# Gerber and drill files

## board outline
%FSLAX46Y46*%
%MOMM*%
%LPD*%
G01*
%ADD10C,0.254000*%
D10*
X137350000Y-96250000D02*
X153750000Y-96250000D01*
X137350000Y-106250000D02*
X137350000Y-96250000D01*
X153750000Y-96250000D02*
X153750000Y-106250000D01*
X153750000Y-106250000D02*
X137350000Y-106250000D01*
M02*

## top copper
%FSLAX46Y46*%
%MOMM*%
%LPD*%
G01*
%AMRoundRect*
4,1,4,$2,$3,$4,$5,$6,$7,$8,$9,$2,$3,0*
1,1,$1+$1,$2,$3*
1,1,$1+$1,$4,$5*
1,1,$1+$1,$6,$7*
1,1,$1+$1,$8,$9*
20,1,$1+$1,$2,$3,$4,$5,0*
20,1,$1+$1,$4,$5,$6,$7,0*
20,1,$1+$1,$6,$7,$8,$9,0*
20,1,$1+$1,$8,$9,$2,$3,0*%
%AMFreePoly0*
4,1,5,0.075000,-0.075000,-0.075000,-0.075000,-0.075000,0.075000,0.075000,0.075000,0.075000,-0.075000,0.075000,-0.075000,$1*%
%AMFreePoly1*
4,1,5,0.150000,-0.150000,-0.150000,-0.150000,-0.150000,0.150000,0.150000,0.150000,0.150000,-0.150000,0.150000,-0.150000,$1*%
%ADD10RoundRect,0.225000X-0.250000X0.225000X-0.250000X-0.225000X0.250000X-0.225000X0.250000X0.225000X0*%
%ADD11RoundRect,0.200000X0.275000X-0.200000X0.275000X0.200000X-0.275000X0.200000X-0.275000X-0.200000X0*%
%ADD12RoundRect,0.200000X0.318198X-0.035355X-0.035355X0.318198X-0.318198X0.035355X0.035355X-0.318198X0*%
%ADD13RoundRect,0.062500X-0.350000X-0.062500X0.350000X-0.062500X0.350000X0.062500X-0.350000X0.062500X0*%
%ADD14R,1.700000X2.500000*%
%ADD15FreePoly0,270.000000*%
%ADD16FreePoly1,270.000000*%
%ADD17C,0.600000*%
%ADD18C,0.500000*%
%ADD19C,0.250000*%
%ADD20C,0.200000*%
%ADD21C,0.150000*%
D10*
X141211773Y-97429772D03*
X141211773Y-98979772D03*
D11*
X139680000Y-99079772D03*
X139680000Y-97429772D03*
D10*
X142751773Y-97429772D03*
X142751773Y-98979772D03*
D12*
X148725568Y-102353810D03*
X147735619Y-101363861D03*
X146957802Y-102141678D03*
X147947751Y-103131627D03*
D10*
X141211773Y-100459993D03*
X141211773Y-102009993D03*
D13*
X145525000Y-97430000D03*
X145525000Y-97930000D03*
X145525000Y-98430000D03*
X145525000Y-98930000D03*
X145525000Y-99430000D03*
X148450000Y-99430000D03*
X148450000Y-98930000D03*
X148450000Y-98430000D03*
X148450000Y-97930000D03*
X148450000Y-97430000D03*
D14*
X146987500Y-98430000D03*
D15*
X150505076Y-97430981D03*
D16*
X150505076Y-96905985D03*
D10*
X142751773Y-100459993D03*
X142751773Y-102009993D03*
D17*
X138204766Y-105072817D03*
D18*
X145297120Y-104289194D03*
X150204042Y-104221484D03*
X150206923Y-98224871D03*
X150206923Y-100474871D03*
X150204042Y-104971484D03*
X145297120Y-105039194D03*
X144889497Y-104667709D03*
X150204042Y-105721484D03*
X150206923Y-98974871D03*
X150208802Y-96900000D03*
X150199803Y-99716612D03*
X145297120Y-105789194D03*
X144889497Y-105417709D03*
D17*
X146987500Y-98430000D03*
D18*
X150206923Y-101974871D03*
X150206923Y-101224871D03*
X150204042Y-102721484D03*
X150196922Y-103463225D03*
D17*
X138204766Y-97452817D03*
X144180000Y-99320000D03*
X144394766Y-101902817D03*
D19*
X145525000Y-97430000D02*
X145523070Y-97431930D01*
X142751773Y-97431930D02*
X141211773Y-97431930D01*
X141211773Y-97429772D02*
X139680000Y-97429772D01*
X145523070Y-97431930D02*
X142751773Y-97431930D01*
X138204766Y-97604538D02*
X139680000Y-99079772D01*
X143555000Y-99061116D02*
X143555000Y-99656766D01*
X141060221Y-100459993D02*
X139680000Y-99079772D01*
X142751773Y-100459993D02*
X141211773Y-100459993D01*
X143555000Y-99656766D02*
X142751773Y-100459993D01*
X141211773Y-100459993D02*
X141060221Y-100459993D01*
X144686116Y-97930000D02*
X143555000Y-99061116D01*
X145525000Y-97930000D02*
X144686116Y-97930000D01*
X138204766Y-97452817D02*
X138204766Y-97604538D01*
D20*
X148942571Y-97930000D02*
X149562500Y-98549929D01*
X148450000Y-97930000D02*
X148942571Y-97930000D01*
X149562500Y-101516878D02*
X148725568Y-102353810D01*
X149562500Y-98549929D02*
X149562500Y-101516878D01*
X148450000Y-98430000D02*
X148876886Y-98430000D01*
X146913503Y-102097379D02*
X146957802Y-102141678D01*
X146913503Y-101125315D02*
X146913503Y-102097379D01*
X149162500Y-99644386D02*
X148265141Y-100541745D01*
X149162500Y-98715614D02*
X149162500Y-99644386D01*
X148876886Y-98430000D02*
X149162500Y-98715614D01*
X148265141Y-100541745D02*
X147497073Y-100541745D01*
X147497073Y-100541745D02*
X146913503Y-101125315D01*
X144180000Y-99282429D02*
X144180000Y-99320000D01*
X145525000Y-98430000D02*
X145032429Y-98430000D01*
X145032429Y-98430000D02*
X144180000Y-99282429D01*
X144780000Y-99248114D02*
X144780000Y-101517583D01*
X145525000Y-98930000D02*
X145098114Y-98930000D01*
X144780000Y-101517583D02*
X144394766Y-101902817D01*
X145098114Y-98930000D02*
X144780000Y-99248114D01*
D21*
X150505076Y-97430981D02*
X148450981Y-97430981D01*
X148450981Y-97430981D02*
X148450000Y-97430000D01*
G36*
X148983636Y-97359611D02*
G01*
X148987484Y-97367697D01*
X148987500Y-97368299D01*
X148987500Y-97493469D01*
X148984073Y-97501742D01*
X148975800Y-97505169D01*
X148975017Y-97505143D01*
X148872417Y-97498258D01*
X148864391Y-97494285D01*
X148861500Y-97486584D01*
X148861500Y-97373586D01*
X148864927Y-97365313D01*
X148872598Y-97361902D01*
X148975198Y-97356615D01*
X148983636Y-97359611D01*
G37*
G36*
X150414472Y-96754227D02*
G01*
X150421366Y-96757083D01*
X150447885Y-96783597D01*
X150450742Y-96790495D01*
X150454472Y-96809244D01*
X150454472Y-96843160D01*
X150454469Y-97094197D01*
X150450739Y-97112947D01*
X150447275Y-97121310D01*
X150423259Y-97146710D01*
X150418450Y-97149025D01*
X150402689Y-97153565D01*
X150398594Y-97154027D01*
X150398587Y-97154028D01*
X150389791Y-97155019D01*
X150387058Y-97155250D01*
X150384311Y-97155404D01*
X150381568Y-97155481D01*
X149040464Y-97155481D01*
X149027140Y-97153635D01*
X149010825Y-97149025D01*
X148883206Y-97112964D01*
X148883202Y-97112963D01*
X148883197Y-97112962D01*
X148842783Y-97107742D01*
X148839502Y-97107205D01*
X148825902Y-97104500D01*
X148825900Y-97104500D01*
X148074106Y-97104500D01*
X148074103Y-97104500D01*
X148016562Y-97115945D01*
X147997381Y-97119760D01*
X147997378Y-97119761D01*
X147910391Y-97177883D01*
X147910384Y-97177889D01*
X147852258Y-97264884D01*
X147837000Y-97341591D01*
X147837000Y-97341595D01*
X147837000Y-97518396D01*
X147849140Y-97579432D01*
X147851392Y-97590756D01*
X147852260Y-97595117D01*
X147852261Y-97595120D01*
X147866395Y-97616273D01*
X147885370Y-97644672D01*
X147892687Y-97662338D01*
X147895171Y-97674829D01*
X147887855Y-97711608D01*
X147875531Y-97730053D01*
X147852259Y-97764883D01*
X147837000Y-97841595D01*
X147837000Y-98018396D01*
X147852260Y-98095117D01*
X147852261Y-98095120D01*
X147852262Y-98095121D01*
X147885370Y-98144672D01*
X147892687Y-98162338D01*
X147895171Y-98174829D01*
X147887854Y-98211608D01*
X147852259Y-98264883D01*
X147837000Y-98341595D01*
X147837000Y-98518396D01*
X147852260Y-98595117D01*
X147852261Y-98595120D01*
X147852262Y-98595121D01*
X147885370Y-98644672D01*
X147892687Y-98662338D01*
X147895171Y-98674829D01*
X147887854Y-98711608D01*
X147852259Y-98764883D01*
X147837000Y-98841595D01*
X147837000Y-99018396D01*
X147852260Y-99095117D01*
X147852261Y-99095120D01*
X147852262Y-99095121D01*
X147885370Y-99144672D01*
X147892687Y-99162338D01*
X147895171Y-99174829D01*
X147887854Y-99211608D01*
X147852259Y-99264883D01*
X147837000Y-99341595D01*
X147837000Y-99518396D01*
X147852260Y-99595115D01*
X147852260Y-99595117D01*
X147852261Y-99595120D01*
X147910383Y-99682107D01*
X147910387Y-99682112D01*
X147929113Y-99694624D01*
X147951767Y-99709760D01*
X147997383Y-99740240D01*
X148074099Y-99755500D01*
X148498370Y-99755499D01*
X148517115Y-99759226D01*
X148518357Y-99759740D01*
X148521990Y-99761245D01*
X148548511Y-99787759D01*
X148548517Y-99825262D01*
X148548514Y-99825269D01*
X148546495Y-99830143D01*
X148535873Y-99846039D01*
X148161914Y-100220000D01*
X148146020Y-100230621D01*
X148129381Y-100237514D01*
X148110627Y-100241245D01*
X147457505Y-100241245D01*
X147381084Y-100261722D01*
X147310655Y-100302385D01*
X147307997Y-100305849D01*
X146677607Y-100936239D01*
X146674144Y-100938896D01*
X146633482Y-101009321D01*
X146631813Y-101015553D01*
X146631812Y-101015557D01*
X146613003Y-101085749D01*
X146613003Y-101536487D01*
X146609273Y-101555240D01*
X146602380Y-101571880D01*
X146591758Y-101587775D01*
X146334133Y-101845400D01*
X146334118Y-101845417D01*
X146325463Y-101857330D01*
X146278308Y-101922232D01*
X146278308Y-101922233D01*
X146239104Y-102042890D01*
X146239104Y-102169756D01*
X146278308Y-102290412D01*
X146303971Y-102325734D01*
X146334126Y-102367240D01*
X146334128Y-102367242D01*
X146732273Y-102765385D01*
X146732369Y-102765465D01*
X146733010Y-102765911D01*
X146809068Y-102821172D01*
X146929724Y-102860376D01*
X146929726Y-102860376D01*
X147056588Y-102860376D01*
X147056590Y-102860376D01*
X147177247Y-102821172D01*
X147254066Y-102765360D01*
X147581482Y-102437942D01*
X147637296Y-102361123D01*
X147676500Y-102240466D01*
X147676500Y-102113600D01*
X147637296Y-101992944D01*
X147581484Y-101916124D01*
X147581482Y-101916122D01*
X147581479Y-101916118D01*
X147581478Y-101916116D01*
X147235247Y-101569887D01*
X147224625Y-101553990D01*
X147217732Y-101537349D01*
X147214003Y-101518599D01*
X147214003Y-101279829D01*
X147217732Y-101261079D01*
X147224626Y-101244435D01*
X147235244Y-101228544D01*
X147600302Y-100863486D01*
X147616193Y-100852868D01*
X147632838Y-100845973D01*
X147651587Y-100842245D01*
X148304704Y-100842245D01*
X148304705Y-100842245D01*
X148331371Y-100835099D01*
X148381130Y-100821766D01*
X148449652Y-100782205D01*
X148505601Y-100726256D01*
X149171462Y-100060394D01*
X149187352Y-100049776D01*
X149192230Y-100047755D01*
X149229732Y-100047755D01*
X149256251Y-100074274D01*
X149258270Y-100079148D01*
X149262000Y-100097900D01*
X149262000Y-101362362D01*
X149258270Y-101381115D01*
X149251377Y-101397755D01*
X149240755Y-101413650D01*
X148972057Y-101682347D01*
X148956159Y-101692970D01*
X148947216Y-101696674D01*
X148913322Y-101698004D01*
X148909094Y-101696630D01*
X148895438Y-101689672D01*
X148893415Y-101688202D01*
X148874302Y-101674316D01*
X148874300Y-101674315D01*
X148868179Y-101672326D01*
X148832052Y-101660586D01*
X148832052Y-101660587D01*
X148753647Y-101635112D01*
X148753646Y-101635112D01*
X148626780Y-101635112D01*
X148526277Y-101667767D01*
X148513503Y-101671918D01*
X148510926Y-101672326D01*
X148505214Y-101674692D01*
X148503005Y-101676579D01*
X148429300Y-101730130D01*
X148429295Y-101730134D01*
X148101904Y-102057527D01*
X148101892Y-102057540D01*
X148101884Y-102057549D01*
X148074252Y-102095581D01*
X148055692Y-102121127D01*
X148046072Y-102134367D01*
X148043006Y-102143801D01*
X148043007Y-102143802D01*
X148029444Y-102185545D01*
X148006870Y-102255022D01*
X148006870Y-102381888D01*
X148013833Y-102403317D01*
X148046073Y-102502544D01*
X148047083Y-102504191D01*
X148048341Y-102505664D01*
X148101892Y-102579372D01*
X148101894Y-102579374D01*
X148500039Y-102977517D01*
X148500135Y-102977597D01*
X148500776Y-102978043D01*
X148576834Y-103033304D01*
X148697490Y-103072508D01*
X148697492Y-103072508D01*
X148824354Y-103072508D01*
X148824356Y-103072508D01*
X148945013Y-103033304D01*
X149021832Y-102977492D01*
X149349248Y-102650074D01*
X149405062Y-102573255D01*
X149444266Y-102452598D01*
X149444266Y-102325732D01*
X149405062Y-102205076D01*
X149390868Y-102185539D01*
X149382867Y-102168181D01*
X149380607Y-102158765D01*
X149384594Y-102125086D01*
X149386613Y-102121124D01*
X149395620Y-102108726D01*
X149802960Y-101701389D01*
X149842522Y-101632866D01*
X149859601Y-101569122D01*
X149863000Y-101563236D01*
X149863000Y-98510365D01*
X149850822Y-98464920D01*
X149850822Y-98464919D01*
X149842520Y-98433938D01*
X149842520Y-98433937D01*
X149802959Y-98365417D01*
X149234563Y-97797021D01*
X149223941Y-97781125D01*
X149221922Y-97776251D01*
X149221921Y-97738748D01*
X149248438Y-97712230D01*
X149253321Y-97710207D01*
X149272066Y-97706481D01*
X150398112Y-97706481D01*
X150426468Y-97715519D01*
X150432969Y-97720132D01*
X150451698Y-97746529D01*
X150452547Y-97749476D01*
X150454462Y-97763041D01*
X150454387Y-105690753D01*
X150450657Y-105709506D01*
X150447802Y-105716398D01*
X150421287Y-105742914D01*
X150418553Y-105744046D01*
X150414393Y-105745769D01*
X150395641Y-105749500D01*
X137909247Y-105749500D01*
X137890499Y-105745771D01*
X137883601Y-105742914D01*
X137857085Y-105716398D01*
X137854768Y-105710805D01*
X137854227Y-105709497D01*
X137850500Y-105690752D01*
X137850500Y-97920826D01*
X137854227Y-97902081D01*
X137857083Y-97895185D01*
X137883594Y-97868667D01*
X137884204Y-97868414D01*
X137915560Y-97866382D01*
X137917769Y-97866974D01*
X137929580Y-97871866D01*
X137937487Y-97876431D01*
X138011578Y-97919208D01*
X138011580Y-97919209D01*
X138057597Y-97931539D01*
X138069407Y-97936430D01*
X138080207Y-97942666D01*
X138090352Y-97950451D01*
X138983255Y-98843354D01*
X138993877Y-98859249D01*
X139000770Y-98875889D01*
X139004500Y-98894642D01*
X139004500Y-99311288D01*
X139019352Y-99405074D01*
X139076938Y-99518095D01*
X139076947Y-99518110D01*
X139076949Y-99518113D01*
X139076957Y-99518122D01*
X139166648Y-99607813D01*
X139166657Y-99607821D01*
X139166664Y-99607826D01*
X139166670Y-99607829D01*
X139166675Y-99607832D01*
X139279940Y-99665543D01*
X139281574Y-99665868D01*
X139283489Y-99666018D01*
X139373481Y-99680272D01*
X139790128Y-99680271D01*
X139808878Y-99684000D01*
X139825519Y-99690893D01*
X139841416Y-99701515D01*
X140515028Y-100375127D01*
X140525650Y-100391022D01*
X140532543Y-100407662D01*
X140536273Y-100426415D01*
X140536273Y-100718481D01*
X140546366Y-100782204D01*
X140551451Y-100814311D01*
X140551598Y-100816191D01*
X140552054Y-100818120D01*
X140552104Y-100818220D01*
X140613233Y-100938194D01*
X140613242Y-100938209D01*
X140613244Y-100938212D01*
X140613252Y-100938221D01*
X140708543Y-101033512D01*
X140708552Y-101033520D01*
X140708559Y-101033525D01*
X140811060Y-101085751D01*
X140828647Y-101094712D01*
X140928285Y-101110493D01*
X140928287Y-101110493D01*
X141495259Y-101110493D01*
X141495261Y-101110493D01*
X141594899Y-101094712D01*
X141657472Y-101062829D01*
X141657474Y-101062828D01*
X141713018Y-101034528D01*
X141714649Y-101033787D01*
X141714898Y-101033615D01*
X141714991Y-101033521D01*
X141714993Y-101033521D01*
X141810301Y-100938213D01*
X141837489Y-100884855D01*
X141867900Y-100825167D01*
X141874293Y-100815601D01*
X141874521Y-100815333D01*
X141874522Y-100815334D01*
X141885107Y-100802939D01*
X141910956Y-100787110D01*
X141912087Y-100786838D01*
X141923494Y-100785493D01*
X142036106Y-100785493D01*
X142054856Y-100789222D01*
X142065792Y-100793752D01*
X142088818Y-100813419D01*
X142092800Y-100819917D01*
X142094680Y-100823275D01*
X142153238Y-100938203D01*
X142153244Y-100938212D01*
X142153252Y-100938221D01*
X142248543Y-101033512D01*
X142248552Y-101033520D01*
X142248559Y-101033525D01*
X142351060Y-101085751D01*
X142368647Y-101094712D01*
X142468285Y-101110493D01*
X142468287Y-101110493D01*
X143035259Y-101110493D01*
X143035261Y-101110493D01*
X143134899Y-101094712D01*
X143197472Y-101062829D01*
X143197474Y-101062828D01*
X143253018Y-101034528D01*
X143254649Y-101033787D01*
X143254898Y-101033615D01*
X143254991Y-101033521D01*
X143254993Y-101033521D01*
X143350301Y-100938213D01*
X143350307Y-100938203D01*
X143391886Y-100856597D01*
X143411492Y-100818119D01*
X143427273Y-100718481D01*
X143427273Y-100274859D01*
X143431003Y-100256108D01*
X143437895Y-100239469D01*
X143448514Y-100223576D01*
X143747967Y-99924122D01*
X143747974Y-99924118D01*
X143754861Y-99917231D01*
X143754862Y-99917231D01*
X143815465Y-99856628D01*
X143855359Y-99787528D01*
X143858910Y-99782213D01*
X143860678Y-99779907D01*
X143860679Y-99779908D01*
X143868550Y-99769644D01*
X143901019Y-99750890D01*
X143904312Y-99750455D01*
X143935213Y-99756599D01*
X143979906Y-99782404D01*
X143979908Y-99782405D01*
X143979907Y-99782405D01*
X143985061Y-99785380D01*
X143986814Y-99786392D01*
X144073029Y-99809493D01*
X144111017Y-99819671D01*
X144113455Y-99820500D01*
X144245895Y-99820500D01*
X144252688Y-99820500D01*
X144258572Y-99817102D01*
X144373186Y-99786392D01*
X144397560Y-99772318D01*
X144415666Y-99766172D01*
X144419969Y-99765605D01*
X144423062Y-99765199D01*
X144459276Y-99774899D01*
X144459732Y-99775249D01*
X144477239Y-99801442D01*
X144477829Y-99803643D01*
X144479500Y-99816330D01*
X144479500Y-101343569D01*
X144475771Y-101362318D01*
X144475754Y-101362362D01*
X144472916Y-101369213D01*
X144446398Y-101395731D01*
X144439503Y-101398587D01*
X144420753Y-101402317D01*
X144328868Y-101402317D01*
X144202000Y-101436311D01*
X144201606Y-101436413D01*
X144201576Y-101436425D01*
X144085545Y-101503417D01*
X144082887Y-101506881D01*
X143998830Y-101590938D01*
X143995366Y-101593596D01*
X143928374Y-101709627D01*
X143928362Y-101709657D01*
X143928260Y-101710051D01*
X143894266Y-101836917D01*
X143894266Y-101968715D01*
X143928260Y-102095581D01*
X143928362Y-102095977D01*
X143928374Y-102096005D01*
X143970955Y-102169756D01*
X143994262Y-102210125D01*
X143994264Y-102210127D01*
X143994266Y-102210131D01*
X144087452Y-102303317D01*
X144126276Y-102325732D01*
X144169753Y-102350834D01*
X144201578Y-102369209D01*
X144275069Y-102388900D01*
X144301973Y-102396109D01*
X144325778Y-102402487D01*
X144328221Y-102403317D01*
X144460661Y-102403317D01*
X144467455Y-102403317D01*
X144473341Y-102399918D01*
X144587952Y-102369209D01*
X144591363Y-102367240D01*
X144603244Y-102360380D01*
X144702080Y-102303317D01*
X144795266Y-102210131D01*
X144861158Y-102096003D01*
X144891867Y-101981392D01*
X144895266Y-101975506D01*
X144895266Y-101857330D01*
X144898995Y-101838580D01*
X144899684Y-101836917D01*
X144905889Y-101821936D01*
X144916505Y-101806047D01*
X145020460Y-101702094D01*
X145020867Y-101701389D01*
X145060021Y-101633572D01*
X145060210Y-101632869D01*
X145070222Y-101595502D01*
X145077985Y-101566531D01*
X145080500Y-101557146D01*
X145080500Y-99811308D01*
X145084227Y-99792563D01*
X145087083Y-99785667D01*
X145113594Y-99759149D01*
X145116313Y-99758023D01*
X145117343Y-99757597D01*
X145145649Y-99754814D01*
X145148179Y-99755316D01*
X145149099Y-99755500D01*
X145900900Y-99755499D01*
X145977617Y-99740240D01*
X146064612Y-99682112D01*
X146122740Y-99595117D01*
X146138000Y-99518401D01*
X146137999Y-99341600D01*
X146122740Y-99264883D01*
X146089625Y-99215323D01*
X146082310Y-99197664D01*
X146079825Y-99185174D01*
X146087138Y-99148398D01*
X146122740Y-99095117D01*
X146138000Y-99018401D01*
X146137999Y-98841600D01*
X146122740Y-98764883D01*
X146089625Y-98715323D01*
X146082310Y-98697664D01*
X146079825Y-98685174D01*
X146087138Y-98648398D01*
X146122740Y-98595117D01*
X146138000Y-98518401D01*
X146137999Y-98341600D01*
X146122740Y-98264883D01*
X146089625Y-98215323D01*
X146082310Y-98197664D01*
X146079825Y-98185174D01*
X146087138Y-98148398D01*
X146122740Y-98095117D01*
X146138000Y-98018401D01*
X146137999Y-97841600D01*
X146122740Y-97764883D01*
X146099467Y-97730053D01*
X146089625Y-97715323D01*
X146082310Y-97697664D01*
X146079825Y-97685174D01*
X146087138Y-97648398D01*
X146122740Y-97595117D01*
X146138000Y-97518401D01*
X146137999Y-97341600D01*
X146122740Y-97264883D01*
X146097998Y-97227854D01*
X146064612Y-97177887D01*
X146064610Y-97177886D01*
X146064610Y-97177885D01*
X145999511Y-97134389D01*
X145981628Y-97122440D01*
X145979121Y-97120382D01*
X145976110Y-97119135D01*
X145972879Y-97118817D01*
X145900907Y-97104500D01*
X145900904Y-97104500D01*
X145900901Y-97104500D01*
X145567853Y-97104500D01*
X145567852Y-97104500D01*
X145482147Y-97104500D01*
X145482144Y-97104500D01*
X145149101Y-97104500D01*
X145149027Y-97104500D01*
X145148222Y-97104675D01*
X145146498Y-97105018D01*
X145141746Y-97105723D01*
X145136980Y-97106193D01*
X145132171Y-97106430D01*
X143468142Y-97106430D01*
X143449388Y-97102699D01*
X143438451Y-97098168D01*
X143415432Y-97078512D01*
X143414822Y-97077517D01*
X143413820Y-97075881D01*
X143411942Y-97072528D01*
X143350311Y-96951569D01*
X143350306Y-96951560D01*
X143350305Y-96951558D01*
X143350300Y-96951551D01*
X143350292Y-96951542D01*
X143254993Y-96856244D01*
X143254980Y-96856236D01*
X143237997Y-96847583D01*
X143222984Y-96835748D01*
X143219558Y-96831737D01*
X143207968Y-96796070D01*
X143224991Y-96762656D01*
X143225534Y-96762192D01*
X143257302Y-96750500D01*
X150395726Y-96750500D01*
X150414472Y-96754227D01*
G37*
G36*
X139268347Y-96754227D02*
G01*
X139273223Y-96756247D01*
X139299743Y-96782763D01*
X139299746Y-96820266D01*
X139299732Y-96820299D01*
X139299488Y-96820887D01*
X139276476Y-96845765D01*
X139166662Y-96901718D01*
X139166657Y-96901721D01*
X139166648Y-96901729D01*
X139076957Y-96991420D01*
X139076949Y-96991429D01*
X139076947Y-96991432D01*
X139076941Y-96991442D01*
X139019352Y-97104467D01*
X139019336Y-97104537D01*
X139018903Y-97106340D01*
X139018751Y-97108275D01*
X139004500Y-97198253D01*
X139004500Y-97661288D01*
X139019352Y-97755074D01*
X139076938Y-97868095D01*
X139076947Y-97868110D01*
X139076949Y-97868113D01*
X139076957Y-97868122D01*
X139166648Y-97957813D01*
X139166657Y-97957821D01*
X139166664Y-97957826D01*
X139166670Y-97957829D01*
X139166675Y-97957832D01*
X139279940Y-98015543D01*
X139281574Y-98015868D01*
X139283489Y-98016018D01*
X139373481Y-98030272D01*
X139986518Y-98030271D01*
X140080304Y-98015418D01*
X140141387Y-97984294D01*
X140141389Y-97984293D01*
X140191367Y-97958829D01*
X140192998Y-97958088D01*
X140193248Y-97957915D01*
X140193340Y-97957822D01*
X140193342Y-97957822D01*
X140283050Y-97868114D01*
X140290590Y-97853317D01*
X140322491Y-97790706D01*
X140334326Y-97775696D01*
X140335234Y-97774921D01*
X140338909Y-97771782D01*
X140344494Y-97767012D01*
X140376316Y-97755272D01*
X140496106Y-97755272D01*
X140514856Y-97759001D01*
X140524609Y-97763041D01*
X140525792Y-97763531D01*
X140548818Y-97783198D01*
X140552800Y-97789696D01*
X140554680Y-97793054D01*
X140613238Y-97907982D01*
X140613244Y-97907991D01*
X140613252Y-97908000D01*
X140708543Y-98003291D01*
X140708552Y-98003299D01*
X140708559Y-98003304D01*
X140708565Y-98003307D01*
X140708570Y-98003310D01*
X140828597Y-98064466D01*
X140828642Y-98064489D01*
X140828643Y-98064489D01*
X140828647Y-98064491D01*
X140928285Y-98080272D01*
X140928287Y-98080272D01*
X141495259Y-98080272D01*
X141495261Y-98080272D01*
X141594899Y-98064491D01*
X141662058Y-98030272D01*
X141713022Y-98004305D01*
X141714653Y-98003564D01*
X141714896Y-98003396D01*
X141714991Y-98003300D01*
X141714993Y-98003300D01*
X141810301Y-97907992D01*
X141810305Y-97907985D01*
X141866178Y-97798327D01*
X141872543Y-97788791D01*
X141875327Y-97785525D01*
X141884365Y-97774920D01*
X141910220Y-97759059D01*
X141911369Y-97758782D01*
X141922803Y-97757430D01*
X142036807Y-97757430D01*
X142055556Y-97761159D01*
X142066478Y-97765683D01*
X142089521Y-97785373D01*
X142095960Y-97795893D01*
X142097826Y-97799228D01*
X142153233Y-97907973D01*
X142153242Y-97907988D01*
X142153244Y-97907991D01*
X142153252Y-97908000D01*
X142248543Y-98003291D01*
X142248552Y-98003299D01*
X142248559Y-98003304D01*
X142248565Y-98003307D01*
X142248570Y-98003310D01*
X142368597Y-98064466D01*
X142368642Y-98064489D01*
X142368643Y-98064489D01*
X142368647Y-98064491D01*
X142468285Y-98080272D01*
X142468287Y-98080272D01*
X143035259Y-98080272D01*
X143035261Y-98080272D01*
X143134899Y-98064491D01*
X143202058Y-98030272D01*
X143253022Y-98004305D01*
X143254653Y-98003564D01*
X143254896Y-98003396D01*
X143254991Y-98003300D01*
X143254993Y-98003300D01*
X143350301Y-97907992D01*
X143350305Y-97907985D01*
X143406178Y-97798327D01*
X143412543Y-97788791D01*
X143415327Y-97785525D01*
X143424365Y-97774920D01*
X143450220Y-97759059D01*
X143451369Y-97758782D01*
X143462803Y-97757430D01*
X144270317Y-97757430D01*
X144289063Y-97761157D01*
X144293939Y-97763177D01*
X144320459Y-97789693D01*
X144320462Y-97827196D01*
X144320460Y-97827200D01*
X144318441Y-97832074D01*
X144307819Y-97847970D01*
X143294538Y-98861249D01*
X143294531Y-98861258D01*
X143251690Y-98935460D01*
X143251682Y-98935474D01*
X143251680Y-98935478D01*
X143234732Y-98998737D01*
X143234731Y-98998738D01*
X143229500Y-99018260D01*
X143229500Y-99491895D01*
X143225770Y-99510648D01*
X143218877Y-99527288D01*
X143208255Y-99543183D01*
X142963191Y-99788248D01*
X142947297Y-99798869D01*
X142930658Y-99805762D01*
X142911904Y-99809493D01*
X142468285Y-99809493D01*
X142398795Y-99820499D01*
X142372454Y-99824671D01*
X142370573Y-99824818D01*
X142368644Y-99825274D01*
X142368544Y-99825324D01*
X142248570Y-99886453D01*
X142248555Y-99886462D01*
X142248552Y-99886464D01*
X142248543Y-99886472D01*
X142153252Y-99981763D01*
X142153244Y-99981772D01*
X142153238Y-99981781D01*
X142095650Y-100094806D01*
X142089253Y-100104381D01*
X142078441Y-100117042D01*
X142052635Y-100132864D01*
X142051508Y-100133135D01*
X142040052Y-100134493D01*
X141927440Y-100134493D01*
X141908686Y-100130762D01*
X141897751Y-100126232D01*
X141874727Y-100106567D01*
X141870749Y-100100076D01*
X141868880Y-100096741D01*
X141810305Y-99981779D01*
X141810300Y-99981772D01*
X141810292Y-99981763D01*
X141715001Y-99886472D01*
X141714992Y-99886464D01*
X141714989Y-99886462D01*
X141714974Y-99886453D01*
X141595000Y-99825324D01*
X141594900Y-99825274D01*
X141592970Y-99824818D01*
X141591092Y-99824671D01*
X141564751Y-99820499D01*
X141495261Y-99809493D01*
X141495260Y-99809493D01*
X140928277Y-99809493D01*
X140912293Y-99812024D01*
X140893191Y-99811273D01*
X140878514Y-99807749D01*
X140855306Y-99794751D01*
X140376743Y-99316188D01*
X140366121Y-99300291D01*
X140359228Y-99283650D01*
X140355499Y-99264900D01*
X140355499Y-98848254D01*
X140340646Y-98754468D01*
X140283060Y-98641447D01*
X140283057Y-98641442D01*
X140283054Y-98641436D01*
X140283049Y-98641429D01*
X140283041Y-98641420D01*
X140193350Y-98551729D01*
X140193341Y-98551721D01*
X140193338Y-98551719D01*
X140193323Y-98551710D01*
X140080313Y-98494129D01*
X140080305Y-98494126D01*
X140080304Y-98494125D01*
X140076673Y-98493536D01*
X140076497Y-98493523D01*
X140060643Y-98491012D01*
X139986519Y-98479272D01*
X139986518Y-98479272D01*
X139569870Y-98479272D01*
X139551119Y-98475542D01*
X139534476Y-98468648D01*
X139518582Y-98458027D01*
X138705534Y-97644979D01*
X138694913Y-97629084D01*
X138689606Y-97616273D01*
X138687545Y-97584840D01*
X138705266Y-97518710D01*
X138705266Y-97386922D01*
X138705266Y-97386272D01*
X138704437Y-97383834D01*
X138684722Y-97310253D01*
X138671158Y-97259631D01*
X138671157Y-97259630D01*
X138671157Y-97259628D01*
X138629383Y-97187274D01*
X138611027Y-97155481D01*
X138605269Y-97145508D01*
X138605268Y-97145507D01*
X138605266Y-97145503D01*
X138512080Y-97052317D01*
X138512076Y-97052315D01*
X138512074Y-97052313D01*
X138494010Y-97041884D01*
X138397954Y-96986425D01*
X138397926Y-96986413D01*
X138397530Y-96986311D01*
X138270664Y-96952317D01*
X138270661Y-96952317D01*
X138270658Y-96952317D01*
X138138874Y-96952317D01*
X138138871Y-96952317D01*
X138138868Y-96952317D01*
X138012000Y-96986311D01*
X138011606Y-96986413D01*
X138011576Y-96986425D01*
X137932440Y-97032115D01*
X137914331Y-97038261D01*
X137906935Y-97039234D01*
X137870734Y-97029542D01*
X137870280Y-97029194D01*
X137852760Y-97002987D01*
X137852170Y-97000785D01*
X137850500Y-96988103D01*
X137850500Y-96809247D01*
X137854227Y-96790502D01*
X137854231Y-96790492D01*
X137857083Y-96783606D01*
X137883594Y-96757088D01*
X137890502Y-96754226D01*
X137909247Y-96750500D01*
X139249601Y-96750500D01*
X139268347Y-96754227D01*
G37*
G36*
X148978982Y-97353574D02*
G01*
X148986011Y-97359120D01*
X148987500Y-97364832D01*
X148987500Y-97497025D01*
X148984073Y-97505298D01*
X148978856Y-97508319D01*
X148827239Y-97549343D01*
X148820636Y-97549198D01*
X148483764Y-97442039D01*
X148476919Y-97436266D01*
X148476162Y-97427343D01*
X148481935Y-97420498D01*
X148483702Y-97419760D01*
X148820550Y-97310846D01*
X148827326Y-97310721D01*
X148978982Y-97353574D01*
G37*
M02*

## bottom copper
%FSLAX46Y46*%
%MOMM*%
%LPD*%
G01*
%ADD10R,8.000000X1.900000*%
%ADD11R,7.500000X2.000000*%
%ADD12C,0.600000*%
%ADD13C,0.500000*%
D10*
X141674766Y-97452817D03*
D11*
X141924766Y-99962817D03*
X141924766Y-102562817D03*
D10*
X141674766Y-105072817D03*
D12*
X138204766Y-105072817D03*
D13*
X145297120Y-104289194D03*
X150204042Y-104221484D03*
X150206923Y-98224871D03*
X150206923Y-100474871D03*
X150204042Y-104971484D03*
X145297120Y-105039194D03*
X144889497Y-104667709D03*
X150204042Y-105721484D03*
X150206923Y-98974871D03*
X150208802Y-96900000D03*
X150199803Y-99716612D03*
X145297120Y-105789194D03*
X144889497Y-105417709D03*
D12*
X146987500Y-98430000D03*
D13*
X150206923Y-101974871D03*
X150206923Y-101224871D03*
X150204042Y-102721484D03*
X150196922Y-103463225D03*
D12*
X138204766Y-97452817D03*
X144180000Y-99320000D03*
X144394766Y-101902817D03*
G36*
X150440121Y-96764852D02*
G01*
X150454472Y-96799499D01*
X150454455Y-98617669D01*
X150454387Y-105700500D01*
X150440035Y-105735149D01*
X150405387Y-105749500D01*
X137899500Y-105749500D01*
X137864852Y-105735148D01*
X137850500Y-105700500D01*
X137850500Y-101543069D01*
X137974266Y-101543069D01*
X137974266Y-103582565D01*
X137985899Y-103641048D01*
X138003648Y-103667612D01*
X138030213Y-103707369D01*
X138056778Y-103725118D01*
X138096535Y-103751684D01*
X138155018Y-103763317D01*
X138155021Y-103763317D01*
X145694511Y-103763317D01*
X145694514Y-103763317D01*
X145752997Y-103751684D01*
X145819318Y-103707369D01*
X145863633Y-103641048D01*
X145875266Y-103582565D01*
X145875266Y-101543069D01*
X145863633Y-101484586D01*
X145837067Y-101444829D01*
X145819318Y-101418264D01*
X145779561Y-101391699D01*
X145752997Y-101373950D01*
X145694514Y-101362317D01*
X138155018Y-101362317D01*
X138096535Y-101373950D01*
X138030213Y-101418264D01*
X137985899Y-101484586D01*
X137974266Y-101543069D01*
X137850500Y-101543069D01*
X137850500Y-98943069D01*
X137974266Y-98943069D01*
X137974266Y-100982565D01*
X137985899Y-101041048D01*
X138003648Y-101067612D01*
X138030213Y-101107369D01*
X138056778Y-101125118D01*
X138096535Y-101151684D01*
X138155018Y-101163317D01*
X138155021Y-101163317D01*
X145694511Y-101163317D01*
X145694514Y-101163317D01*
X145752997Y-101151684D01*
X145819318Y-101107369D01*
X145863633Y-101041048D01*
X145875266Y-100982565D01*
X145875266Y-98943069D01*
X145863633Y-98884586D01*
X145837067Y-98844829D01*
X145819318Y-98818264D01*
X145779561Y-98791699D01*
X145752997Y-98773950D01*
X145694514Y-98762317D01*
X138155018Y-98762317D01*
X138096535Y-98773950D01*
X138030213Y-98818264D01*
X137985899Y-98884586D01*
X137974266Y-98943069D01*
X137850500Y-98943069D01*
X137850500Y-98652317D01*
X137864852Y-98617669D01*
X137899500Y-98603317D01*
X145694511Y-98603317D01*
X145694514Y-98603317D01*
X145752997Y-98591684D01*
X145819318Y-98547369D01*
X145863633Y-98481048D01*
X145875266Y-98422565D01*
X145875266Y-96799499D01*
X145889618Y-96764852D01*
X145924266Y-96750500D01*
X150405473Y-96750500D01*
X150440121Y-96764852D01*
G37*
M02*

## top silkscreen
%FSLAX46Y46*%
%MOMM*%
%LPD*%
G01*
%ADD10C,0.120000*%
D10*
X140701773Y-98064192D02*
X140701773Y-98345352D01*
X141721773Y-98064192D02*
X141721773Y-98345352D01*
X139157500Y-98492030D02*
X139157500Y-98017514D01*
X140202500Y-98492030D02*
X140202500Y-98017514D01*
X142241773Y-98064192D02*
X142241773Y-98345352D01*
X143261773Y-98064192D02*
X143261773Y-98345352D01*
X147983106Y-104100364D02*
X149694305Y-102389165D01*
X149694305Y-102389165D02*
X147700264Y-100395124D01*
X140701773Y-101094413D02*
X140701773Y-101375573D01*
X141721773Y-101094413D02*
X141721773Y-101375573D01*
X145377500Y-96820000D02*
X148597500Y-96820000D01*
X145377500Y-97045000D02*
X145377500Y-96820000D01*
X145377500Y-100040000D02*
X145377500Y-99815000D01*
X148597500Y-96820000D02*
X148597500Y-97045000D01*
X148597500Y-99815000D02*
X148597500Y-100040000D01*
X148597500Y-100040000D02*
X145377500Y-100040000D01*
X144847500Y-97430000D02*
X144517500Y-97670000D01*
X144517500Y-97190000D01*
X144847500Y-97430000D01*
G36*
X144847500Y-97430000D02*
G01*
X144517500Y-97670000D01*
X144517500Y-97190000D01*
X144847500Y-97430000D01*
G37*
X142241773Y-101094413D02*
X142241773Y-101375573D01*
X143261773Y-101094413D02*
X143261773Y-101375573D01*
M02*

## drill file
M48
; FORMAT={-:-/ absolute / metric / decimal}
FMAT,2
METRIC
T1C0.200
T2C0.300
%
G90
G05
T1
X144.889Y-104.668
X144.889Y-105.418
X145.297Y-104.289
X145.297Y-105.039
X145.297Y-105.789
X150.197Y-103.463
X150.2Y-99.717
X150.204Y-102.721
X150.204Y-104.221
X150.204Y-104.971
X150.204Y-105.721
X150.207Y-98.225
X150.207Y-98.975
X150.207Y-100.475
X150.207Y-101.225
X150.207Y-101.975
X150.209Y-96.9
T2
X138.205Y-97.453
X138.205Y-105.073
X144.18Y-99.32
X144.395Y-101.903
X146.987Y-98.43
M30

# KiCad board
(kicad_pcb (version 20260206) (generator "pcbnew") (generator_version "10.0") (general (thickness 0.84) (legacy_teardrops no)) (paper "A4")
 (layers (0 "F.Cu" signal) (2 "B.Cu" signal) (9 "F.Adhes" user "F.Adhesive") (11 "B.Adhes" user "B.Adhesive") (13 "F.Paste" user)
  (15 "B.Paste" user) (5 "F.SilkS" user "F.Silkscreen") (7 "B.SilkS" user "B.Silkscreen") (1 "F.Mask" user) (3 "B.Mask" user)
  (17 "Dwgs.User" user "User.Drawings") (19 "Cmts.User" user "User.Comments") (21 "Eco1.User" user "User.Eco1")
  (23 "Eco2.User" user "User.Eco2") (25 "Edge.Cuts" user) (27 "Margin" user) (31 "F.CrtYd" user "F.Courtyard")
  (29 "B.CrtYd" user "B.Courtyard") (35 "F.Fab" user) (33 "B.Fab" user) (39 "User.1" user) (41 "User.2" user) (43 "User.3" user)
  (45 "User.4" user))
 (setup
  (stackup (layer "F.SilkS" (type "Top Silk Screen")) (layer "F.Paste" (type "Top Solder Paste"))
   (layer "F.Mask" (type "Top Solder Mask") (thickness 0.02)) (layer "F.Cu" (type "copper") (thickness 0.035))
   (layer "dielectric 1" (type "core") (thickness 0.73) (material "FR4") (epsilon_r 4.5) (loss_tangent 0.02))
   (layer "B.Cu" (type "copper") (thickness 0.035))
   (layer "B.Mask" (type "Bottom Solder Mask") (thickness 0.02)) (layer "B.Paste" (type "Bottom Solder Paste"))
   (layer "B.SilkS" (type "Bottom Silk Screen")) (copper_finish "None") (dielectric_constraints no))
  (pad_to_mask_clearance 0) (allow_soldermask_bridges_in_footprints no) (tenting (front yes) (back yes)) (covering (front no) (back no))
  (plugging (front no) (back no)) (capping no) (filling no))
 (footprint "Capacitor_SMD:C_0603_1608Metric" (layer "F.Cu") (at 141.211773 98.204772 -90)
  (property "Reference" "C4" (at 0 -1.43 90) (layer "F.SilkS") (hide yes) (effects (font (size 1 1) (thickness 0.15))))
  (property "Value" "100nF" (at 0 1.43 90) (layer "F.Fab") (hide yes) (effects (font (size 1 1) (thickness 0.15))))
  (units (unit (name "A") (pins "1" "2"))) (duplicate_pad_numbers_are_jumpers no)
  (fp_line (start -0.14058 0.51) (end 0.14058 0.51) (stroke (width 0.12) (type solid)) (layer "F.SilkS"))
  (fp_line (start -0.14058 -0.51) (end 0.14058 -0.51) (stroke (width 0.12) (type solid)) (layer "F.SilkS"))
  (pad "1" smd roundrect (at -0.775 0 270) (size 0.9 0.95) (layers "F.Cu" "F.Mask" "F.Paste") (roundrect_rratio 0.25) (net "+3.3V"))
  (pad "2" smd roundrect (at 0.775 0 270) (size 0.9 0.95) (layers "F.Cu" "F.Mask" "F.Paste") (roundrect_rratio 0.25) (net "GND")))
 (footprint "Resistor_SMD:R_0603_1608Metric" (layer "F.Cu") (at 139.68 98.254772 90)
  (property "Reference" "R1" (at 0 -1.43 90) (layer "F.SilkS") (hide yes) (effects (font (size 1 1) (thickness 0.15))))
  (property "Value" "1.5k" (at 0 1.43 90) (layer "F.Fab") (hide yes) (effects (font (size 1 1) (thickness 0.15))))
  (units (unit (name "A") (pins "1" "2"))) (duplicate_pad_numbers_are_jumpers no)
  (fp_line (start -0.237258 -0.5225) (end 0.237258 -0.5225) (stroke (width 0.12) (type solid)) (layer "F.SilkS"))
  (fp_line (start -0.237258 0.5225) (end 0.237258 0.5225) (stroke (width 0.12) (type solid)) (layer "F.SilkS"))
  (pad "1" smd roundrect (at -0.825 0 90) (size 0.8 0.95) (layers "F.Cu" "F.Mask" "F.Paste") (roundrect_rratio 0.25) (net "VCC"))
  (pad "2" smd roundrect (at 0.825 0 90) (size 0.8 0.95) (layers "F.Cu" "F.Mask" "F.Paste") (roundrect_rratio 0.25) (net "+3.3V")))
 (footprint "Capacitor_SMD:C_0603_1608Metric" (layer "F.Cu") (at 142.751773 98.204772 -90)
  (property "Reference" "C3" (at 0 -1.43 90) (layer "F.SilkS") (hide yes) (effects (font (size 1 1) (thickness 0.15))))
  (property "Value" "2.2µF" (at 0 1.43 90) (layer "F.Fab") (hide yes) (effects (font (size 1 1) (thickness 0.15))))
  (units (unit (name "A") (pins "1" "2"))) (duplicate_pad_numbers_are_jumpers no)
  (fp_line (start -0.14058 0.51) (end 0.14058 0.51) (stroke (width 0.12) (type solid)) (layer "F.SilkS"))
  (fp_line (start -0.14058 -0.51) (end 0.14058 -0.51) (stroke (width 0.12) (type solid)) (layer "F.SilkS"))
  (pad "1" smd roundrect (at -0.775 0 270) (size 0.9 0.95) (layers "F.Cu" "F.Mask" "F.Paste") (roundrect_rratio 0.25) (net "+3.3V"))
  (pad "2" smd roundrect (at 0.775 0 270) (size 0.9 0.95) (layers "F.Cu" "F.Mask" "F.Paste") (roundrect_rratio 0.25) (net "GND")))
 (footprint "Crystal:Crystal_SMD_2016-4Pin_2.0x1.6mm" (layer "F.Cu") (at 147.841685 102.247744 135)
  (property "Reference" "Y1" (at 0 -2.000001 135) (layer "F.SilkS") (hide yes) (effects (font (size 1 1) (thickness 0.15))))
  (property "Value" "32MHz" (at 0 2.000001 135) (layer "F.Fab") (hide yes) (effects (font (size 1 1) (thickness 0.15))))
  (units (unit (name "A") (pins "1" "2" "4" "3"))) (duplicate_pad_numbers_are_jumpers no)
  (fp_line (start -1.41 -1.21) (end -1.41 1.21) (stroke (width 0.12) (type solid)) (layer "F.SilkS"))
  (fp_line (start -1.41 1.21) (end 1.41 1.21) (stroke (width 0.12) (type solid)) (layer "F.SilkS"))
  (pad "1" smd roundrect (at -0.7 0.55 135) (size 0.9 0.8) (layers "F.Cu" "F.Mask" "F.Paste") (roundrect_rratio 0.25) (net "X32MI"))
  (pad "2" smd roundrect (at 0.7 0.55 135) (size 0.9 0.8) (layers "F.Cu" "F.Mask" "F.Paste") (roundrect_rratio 0.25) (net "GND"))
  (pad "3" smd roundrect (at 0.7 -0.55 135) (size 0.9 0.8) (layers "F.Cu" "F.Mask" "F.Paste") (roundrect_rratio 0.25) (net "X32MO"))
  (pad "4" smd roundrect (at -0.7 -0.55 135) (size 0.9 0.8) (layers "F.Cu" "F.Mask" "F.Paste") (roundrect_rratio 0.25) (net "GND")))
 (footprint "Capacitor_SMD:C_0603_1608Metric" (layer "F.Cu") (at 141.211773 101.234993 -90)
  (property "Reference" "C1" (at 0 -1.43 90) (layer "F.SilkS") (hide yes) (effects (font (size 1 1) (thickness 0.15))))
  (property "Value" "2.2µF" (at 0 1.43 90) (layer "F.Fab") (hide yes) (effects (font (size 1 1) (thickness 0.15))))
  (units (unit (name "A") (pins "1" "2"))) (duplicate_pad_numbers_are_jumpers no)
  (fp_line (start -0.14058 0.51) (end 0.14058 0.51) (stroke (width 0.12) (type solid)) (layer "F.SilkS"))
  (fp_line (start -0.14058 -0.51) (end 0.14058 -0.51) (stroke (width 0.12) (type solid)) (layer "F.SilkS"))
  (pad "1" smd roundrect (at -0.775 0 270) (size 0.9 0.95) (layers "F.Cu" "F.Mask" "F.Paste") (roundrect_rratio 0.25) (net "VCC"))
  (pad "2" smd roundrect (at 0.775 0 270) (size 0.9 0.95) (layers "F.Cu" "F.Mask" "F.Paste") (roundrect_rratio 0.25) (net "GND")))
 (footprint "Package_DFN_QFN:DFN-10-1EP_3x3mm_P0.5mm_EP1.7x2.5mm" (layer "F.Cu") (at 146.9875 98.43)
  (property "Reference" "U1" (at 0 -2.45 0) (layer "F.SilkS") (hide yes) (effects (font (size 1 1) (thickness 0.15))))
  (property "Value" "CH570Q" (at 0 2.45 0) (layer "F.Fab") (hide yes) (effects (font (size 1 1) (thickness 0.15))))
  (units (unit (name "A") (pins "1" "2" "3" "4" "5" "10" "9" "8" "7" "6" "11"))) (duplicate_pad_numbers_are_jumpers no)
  (fp_line (start -1.61 -1.61) (end 1.61 -1.61) (stroke (width 0.12) (type solid)) (layer "F.SilkS"))
  (fp_line (start -1.61 -1.385) (end -1.61 -1.61) (stroke (width 0.12) (type solid)) (layer "F.SilkS"))
  (fp_line (start -1.61 1.61) (end -1.61 1.385) (stroke (width 0.12) (type solid)) (layer "F.SilkS"))
  (fp_line (start 1.61 -1.61) (end 1.61 -1.385) (stroke (width 0.12) (type solid)) (layer "F.SilkS"))
  (fp_line (start 1.61 1.385) (end 1.61 1.61) (stroke (width 0.12) (type solid)) (layer "F.SilkS"))
  (fp_line (start 1.61 1.61) (end -1.61 1.61) (stroke (width 0.12) (type solid)) (layer "F.SilkS"))
  (fp_poly (pts (xy -2.14 -1) (xy -2.47 -0.76) (xy -2.47 -1.24)) (stroke (width 0.12) (type solid)) (fill yes) (layer "F.SilkS"))
  (pad "" smd roundrect (at -0.425 -0.625) (size 0.69 1.01) (layers "F.Paste") (roundrect_rratio 0.25))
  (pad "" smd roundrect (at -0.425 0.625) (size 0.69 1.01) (layers "F.Paste") (roundrect_rratio 0.25))
  (pad "" smd roundrect (at 0.425 -0.625) (size 0.69 1.01) (layers "F.Paste") (roundrect_rratio 0.25))
  (pad "" smd roundrect (at 0.425 0.625) (size 0.69 1.01) (layers "F.Paste") (roundrect_rratio 0.25))
  (pad "1" smd roundrect (at -1.4625 -1) (size 0.825 0.25) (layers "F.Cu" "F.Mask" "F.Paste") (roundrect_rratio 0.25) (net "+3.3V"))
  (pad "2" smd roundrect (at -1.4625 -0.5) (size 0.825 0.25) (layers "F.Cu" "F.Mask" "F.Paste") (roundrect_rratio 0.25) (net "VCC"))
  (pad "3" smd roundrect (at -1.4625 0) (size 0.825 0.25) (layers "F.Cu" "F.Mask" "F.Paste") (roundrect_rratio 0.25) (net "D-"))
  (pad "4" smd roundrect (at -1.4625 0.5) (size 0.825 0.25) (layers "F.Cu" "F.Mask" "F.Paste") (roundrect_rratio 0.25) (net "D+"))
  (pad "5" smd roundrect (at -1.4625 1) (size 0.825 0.25) (layers "F.Cu" "F.Mask" "F.Paste") (roundrect_rratio 0.25)
   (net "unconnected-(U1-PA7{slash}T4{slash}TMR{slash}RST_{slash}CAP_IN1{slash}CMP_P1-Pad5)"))
  (pad "6" smd roundrect (at 1.4625 1) (size 0.825 0.25) (layers "F.Cu" "F.Mask" "F.Paste") (roundrect_rratio 0.25)
   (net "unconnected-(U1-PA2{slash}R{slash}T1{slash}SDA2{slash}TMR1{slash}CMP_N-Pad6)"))
  (pad "7" smd roundrect (at 1.4625 0.5) (size 0.825 0.25) (layers "F.Cu" "F.Mask" "F.Paste") (roundrect_rratio 0.25)
   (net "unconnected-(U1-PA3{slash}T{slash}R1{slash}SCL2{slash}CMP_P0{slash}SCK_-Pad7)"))
  (pad "8" smd roundrect (at 1.4625 0) (size 0.825 0.25) (layers "F.Cu" "F.Mask" "F.Paste") (roundrect_rratio 0.25) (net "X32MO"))
  (pad "9" smd roundrect (at 1.4625 -0.5) (size 0.825 0.25) (layers "F.Cu" "F.Mask" "F.Paste") (roundrect_rratio 0.25) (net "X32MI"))
  (pad "10" smd roundrect (at 1.4625 -1) (size 0.825 0.25) (layers "F.Cu" "F.Mask" "F.Paste") (roundrect_rratio 0.25) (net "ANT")
   (teardrops (best_length_ratio 0.5) (max_length 1) (best_width_ratio 1) (max_width 2) (curved_edges no) (filter_ratio 0.9) (enabled yes)
    (allow_two_segments yes) (prefer_zone_connections yes)))
  (pad "11" smd rect (at 0 0) (size 1.7 2.5) (layers "F.Cu" "F.Mask") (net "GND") (zone_connect 2)))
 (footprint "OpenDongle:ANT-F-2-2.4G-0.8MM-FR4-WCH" (layer "F.Cu") (at 151.800076 101.240981 -90)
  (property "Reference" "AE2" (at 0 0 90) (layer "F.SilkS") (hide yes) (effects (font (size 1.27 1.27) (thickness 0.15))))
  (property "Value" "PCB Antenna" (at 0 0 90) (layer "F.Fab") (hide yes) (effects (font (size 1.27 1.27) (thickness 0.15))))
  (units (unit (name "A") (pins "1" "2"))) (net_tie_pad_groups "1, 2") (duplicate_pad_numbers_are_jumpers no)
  (pad "1" smd custom (at -3.81 1.295 270) (size 0.15 0.15) (layers "F.Cu") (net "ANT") (solder_mask_margin 0.1016)
   (options (clearance outline) (anchor rect)) (primitives)
   (teardrops (best_length_ratio 0.5) (max_length 1) (best_width_ratio 1) (max_width 2) (curved_edges no) (filter_ratio 0.9) (enabled yes)
    (allow_two_segments yes) (prefer_zone_connections yes)))
  (pad "2" smd custom (at -4.334996 1.295 270) (size 0.3 0.3) (layers "F.Cu") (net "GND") (solder_mask_margin 0.1016)
   (options (clearance outline) (anchor rect)) (primitives)))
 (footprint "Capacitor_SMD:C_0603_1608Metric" (layer "F.Cu") (at 142.751773 101.234993 -90)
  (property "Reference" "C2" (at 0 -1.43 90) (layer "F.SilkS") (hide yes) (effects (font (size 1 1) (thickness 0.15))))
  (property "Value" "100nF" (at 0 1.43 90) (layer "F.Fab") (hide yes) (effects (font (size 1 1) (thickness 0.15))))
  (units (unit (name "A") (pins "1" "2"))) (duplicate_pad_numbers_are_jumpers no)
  (fp_line (start -0.14058 0.51) (end 0.14058 0.51) (stroke (width 0.12) (type solid)) (layer "F.SilkS"))
  (fp_line (start -0.14058 -0.51) (end 0.14058 -0.51) (stroke (width 0.12) (type solid)) (layer "F.SilkS"))
  (pad "1" smd roundrect (at -0.775 0 270) (size 0.9 0.95) (layers "F.Cu" "F.Mask" "F.Paste") (roundrect_rratio 0.25) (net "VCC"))
  (pad "2" smd roundrect (at 0.775 0 270) (size 0.9 0.95) (layers "F.Cu" "F.Mask" "F.Paste") (roundrect_rratio 0.25) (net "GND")))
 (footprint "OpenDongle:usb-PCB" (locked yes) (layer "B.Cu") (at 136.774766 101.262817 90)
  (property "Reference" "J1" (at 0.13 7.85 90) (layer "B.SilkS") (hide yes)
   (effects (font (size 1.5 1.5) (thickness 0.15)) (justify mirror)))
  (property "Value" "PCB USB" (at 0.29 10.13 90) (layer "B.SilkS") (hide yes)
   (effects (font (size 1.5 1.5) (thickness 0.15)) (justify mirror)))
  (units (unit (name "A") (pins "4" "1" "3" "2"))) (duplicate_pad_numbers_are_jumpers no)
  (pad "1" connect rect (at 3.81 4.9 90) (size 1.9 8) (layers "B.Cu" "B.Mask") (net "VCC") (thermal_bridge_angle 45))
  (pad "2" connect rect (at 1.3 5.15 90) (size 2 7.5) (layers "B.Cu" "B.Mask") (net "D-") (thermal_bridge_angle 45))
  (pad "3" connect rect (at -1.3 5.15 90) (size 2 7.5) (layers "B.Cu" "B.Mask") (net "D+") (thermal_bridge_angle 45))
  (pad "4" connect rect (at -3.81 4.9 90) (size 1.9 8) (layers "B.Cu" "B.Mask") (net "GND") (thermal_bridge_angle 45)))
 (gr_line (start 137.35 96.25) (end 153.75 96.25) (stroke (width 0.254) (type default)) (layer "Edge.Cuts"))
 (gr_line (start 137.35 106.25) (end 137.35 96.25) (stroke (width 0.254) (type default)) (layer "Edge.Cuts"))
 (gr_line (start 153.75 96.25) (end 153.75 106.25) (stroke (width 0.254) (type default)) (layer "Edge.Cuts"))
 (gr_line (start 153.75 106.25) (end 137.35 106.25) (stroke (width 0.254) (type default)) (locked yes) (layer "Edge.Cuts"))
 (segment (start 145.525 97.43) (end 145.52307 97.43193) (width 0.25) (layer "F.Cu") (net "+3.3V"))
 (segment (start 142.751773 97.43193) (end 141.211773 97.43193) (width 0.25) (layer "F.Cu") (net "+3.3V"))
 (segment (start 141.211773 97.429772) (end 139.68 97.429772) (width 0.25) (layer "F.Cu") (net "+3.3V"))
 (segment (start 145.52307 97.43193) (end 142.751773 97.43193) (width 0.25) (layer "F.Cu") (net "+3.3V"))
 (via (at 138.204766 105.072817) (size 0.6) (drill 0.3) (layers "F.Cu" "B.Cu") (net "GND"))
 (via (at 145.29712 104.289194) (size 0.5) (drill 0.2) (layers "F.Cu" "B.Cu") (free yes) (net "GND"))
 (via (at 150.204042 104.221484) (size 0.5) (drill 0.2) (layers "F.Cu" "B.Cu") (free yes) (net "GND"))
 (via (at 150.206923 98.224871) (size 0.5) (drill 0.2) (layers "F.Cu" "B.Cu") (free yes) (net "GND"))
 (via (at 150.206923 100.474871) (size 0.5) (drill 0.2) (layers "F.Cu" "B.Cu") (free yes) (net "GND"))
 (via (at 150.204042 104.971484) (size 0.5) (drill 0.2) (layers "F.Cu" "B.Cu") (free yes) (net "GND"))
 (via (at 145.29712 105.039194) (size 0.5) (drill 0.2) (layers "F.Cu" "B.Cu") (free yes) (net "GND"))
 (via (at 144.889497 104.667709) (size 0.5) (drill 0.2) (layers "F.Cu" "B.Cu") (free yes) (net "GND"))
 (via (at 150.204042 105.721484) (size 0.5) (drill 0.2) (layers "F.Cu" "B.Cu") (free yes) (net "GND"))
 (via (at 150.206923 98.974871) (size 0.5) (drill 0.2) (layers "F.Cu" "B.Cu") (free yes) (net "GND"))
 (via (at 150.208802 96.9) (size 0.5) (drill 0.2) (layers "F.Cu" "B.Cu") (free yes) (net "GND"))
 (via (at 150.199803 99.716612) (size 0.5) (drill 0.2) (layers "F.Cu" "B.Cu") (free yes) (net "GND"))
 (via (at 145.29712 105.789194) (size 0.5) (drill 0.2) (layers "F.Cu" "B.Cu") (free yes) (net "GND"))
 (via (at 144.889497 105.417709) (size 0.5) (drill 0.2) (layers "F.Cu" "B.Cu") (free yes) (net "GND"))
 (via (at 146.9875 98.43) (size 0.6) (drill 0.3) (layers "F.Cu" "B.Cu") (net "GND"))
 (via (at 150.206923 101.974871) (size 0.5) (drill 0.2) (layers "F.Cu" "B.Cu") (free yes) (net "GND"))
 (via (at 150.206923 101.224871) (size 0.5) (drill 0.2) (layers "F.Cu" "B.Cu") (free yes) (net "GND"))
 (via (at 150.204042 102.721484) (size 0.5) (drill 0.2) (layers "F.Cu" "B.Cu") (free yes) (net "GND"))
 (via (at 150.196922 103.463225) (size 0.5) (drill 0.2) (layers "F.Cu" "B.Cu") (free yes) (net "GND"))
 (segment (start 138.204766 97.604538) (end 139.68 99.079772) (width 0.25) (layer "F.Cu") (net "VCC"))
 (segment (start 143.555 99.061116) (end 143.555 99.656766) (width 0.25) (layer "F.Cu") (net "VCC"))
 (segment (start 141.060221 100.459993) (end 139.68 99.079772) (width 0.25) (layer "F.Cu") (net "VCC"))
 (segment (start 142.751773 100.459993) (end 141.211773 100.459993) (width 0.25) (layer "F.Cu") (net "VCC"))
 (segment (start 143.555 99.656766) (end 142.751773 100.459993) (width 0.25) (layer "F.Cu") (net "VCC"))
 (segment (start 141.211773 100.459993) (end 141.060221 100.459993) (width 0.25) (layer "F.Cu") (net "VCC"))
 (segment (start 144.686116 97.93) (end 143.555 99.061116) (width 0.25) (layer "F.Cu") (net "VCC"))
 (segment (start 145.525 97.93) (end 144.686116 97.93) (width 0.25) (layer "F.Cu") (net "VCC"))
 (segment (start 138.204766 97.452817) (end 138.204766 97.604538) (width 0.25) (layer "F.Cu") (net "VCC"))
 (via (at 138.204766 97.452817) (size 0.6) (drill 0.3) (layers "F.Cu" "B.Cu") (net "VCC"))
 (segment (start 148.942571 97.93) (end 149.5625 98.549929) (width 0.2) (layer "F.Cu") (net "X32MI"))
 (segment (start 148.45 97.93) (end 148.942571 97.93) (width 0.2) (layer "F.Cu") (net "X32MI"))
 (segment (start 149.5625 101.516878) (end 148.725568 102.35381) (width 0.2) (layer "F.Cu") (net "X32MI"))
 (segment (start 149.5625 98.549929) (end 149.5625 101.516878) (width 0.2) (layer "F.Cu") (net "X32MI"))
 (segment (start 148.45 98.43) (end 148.876886 98.43) (width 0.2) (layer "F.Cu") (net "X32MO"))
 (segment (start 146.913503 102.097379) (end 146.957802 102.141678) (width 0.2) (layer "F.Cu") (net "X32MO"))
 (segment (start 146.913503 101.125315) (end 146.913503 102.097379) (width 0.2) (layer "F.Cu") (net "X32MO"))
 (segment (start 149.1625 99.644386) (end 148.265141 100.541745) (width 0.2) (layer "F.Cu") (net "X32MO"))
 (segment (start 149.1625 98.715614) (end 149.1625 99.644386) (width 0.2) (layer "F.Cu") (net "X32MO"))
 (segment (start 148.876886 98.43) (end 149.1625 98.715614) (width 0.2) (layer "F.Cu") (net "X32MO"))
 (segment (start 148.265141 100.541745) (end 147.497073 100.541745) (width 0.2) (layer "F.Cu") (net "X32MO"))
 (segment (start 147.497073 100.541745) (end 146.913503 101.125315) (width 0.2) (layer "F.Cu") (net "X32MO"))
 (segment (start 144.18 99.282429) (end 144.18 99.32) (width 0.2) (layer "F.Cu") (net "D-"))
 (segment (start 145.525 98.43) (end 145.032429 98.43) (width 0.2) (layer "F.Cu") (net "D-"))
 (segment (start 145.032429 98.43) (end 144.18 99.282429) (width 0.2) (layer "F.Cu") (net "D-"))
 (via (at 144.18 99.32) (size 0.6) (drill 0.3) (layers "F.Cu" "B.Cu") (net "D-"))
 (segment (start 144.78 99.248114) (end 144.78 101.517583) (width 0.2) (layer "F.Cu") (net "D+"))
 (segment (start 145.525 98.93) (end 145.098114 98.93) (width 0.2) (layer "F.Cu") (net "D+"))
 (segment (start 144.78 101.517583) (end 144.394766 101.902817) (width 0.2) (layer "F.Cu") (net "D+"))
 (segment (start 145.098114 98.93) (end 144.78 99.248114) (width 0.2) (layer "F.Cu") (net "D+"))
 (via (at 144.394766 101.902817) (size 0.6) (drill 0.3) (layers "F.Cu" "B.Cu") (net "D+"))
 (segment (start 150.505076 97.430981) (end 148.450981 97.430981) (width 0.15) (layer "F.Cu") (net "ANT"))
 (segment (start 148.450981 97.430981) (end 148.45 97.43) (width 0.15) (layer "F.Cu") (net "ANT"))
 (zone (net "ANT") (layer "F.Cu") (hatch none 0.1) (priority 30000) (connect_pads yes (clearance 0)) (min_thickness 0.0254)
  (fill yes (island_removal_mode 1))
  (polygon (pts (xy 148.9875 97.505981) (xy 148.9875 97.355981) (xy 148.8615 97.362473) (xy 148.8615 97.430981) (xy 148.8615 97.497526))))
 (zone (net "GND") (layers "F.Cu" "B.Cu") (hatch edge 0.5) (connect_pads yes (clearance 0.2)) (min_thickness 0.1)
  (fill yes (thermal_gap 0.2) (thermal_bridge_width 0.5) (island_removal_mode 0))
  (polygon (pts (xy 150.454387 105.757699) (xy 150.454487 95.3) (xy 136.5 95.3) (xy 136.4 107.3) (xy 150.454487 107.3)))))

